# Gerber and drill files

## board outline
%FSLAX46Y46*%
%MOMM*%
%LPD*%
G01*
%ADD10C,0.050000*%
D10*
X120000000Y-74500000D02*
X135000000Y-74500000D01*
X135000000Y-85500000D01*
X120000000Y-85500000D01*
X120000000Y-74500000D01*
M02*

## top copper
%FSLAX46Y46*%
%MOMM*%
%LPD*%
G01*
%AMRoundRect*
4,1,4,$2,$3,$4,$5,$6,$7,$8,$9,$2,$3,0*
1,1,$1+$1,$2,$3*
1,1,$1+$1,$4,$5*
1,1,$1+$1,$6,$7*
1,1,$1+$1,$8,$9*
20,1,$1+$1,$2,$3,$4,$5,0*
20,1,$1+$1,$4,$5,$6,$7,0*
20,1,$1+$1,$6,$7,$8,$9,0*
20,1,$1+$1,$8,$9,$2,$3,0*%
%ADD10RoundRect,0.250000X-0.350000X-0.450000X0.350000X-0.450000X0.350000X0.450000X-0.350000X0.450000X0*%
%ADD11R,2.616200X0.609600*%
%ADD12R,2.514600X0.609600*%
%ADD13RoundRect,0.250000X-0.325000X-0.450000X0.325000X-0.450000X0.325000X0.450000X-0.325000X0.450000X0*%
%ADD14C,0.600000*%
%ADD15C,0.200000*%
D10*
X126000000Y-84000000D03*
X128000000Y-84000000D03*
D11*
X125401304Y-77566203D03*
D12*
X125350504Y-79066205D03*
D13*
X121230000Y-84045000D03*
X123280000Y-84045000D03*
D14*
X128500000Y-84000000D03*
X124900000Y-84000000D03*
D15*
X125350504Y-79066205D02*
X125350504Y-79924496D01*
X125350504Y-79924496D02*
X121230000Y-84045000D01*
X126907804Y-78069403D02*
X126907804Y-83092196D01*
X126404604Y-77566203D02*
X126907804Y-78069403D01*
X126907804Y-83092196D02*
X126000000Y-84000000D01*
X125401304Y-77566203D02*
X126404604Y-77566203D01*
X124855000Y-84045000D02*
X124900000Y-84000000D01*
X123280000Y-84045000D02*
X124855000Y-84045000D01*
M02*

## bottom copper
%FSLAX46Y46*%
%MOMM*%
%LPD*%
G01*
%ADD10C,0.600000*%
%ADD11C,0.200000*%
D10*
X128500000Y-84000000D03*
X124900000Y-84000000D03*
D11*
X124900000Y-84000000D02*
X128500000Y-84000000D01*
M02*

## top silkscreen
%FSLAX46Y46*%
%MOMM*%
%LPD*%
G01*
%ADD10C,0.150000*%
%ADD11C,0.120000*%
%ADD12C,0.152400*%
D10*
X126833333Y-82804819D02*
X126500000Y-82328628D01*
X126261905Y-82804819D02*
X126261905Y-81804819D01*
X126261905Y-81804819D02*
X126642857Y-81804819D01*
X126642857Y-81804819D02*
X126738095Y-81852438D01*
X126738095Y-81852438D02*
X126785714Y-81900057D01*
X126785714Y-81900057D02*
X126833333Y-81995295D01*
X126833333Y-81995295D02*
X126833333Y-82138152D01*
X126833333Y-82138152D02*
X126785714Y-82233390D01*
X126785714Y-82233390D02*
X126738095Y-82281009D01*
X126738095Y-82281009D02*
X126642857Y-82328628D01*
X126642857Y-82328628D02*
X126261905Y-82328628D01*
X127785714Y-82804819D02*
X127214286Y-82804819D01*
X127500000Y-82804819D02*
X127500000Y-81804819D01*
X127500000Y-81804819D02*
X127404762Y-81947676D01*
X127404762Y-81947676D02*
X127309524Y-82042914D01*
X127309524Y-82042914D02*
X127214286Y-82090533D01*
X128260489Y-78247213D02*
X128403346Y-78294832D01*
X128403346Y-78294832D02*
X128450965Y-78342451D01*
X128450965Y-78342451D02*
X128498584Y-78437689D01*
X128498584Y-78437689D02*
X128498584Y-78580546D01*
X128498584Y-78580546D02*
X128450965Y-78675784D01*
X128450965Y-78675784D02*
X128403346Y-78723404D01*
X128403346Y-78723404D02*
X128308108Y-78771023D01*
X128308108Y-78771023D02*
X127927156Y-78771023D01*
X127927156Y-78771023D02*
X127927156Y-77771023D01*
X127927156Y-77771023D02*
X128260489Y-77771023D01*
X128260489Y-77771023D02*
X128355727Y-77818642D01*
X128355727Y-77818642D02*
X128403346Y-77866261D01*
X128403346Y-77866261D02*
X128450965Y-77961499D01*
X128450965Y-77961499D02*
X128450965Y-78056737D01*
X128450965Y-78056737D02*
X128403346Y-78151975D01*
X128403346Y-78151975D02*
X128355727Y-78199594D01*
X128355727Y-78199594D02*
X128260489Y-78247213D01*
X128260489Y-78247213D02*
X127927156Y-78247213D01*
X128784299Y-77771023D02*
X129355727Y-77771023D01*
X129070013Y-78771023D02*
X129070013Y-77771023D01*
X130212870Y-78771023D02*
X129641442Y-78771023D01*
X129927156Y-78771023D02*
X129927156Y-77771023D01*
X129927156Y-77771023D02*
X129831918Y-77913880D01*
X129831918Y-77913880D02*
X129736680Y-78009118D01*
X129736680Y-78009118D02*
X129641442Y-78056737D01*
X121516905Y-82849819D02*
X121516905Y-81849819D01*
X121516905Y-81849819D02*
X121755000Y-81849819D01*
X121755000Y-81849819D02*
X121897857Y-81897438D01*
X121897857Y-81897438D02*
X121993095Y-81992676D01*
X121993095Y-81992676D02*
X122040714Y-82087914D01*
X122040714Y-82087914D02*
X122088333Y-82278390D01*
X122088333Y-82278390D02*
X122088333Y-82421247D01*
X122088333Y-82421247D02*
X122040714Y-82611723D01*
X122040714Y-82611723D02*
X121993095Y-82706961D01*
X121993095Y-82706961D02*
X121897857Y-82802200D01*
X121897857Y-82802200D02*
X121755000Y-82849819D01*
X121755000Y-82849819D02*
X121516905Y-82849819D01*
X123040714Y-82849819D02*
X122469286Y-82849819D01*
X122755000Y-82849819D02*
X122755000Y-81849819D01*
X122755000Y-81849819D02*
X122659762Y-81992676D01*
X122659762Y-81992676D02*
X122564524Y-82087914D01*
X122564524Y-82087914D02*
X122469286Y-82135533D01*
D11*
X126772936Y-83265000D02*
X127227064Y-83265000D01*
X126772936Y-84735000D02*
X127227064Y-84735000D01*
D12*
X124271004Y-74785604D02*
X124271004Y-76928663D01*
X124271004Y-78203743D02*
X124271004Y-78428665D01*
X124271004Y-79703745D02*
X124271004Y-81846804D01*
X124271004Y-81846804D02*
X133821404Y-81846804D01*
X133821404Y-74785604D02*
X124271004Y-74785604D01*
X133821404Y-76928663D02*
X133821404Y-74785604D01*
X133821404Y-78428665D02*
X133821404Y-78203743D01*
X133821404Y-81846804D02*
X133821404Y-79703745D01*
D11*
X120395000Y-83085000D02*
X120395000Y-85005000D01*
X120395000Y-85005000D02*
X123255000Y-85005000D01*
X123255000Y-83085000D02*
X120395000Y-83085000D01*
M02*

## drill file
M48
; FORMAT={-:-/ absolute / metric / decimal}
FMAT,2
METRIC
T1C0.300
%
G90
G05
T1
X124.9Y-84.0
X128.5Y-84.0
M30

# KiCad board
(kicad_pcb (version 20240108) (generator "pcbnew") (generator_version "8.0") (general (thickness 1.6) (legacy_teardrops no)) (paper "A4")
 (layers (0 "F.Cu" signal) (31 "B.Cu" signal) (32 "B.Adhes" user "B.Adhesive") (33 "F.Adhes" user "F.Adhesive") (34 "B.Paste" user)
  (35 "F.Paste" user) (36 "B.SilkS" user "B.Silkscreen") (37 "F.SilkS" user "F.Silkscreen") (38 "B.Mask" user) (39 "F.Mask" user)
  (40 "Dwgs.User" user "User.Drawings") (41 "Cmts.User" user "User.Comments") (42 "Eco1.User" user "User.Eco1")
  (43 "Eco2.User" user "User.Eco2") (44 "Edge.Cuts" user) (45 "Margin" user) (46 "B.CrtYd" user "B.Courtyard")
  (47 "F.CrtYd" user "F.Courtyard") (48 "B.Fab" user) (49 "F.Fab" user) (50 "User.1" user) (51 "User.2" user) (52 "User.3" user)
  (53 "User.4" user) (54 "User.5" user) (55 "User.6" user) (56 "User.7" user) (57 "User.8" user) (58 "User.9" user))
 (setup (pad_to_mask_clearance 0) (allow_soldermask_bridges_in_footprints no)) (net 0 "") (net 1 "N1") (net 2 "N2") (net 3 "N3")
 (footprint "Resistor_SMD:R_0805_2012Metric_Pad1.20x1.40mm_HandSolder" (layer "F.Cu") (at 127 84)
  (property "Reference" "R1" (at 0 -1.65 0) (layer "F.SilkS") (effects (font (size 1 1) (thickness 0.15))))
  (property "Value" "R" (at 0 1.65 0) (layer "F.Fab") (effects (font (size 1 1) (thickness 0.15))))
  (fp_line (start -0.227064 -0.735) (end 0.227064 -0.735) (stroke (width 0.12) (type solid)) (layer "F.SilkS"))
  (fp_line (start -0.227064 0.735) (end 0.227064 0.735) (stroke (width 0.12) (type solid)) (layer "F.SilkS"))
  (pad "1" smd roundrect (at -1 0) (size 1.2 1.4) (layers "F.Cu" "F.Paste" "F.Mask") (roundrect_rratio 0.208333) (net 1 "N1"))
  (pad "2" smd roundrect (at 1 0) (size 1.2 1.4) (layers "F.Cu" "F.Paste" "F.Mask") (roundrect_rratio 0.208333) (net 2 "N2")))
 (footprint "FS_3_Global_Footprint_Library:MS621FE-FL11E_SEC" (layer "F.Cu") (at 129.046204 78.316204)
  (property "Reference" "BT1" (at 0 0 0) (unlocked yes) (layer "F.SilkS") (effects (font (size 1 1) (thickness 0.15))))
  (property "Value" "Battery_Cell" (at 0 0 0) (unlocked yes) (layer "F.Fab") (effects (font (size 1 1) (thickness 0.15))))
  (fp_line (start -4.7752 -3.5306) (end -4.7752 -1.387541) (stroke (width 0.1524) (type solid)) (layer "F.SilkS"))
  (fp_line (start -4.7752 -0.112461) (end -4.7752 0.112461) (stroke (width 0.1524) (type solid)) (layer "F.SilkS"))
  (fp_line (start -4.7752 1.387541) (end -4.7752 3.5306) (stroke (width 0.1524) (type solid)) (layer "F.SilkS"))
  (fp_line (start -4.7752 3.5306) (end 4.7752 3.5306) (stroke (width 0.1524) (type solid)) (layer "F.SilkS"))
  (fp_line (start 4.7752 -3.5306) (end -4.7752 -3.5306) (stroke (width 0.1524) (type solid)) (layer "F.SilkS"))
  (fp_line (start 4.7752 -1.387541) (end 4.7752 -3.5306) (stroke (width 0.1524) (type solid)) (layer "F.SilkS"))
  (fp_line (start 4.7752 0.112461) (end 4.7752 -0.112461) (stroke (width 0.1524) (type solid)) (layer "F.SilkS"))
  (fp_line (start 4.7752 3.5306) (end 4.7752 1.387541) (stroke (width 0.1524) (type solid)) (layer "F.SilkS"))
  (pad "1" smd rect (at -3.6449 -0.750001) (size 2.6162 0.6096) (layers "F.Cu" "F.Paste" "F.Mask") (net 1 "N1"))
  (pad "2" smd rect (at -3.6957 0.750001) (size 2.5146 0.6096) (layers "F.Cu" "F.Paste" "F.Mask") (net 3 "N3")))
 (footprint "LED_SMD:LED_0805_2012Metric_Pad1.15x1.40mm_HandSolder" (layer "F.Cu") (at 122.255 84.045)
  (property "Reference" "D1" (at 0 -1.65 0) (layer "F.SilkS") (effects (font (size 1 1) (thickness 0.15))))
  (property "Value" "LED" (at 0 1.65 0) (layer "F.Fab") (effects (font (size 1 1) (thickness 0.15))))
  (fp_line (start -1.86 -0.96) (end -1.86 0.96) (stroke (width 0.12) (type solid)) (layer "F.SilkS"))
  (fp_line (start -1.86 0.96) (end 1 0.96) (stroke (width 0.12) (type solid)) (layer "F.SilkS"))
  (fp_line (start 1 -0.96) (end -1.86 -0.96) (stroke (width 0.12) (type solid)) (layer "F.SilkS"))
  (pad "1" smd roundrect (at -1.025 0) (size 1.15 1.4) (layers "F.Cu" "F.Paste" "F.Mask") (roundrect_rratio 0.217391) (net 3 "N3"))
  (pad "2" smd roundrect (at 1.025 0) (size 1.15 1.4) (layers "F.Cu" "F.Paste" "F.Mask") (roundrect_rratio 0.217391) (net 2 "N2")))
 (gr_rect (start 120 74.5) (end 135 85.5) (stroke (width 0.05) (type default)) (fill none) (layer "Edge.Cuts"))
 (segment (start 125.350504 79.066205) (end 125.350504 79.924496) (width 0.2) (layer "F.Cu") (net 3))
 (segment (start 125.350504 79.924496) (end 121.23 84.045) (width 0.2) (layer "F.Cu") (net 3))
 (segment (start 126.907804 78.069403) (end 126.907804 83.092196) (width 0.2) (layer "F.Cu") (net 1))
 (segment (start 126.404604 77.566203) (end 126.907804 78.069403) (width 0.2) (layer "F.Cu") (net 1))
 (segment (start 126.907804 83.092196) (end 126 84) (width 0.2) (layer "F.Cu") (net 1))
 (segment (start 125.401304 77.566203) (end 126.404604 77.566203) (width 0.2) (layer "F.Cu") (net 1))
 (segment (start 124.855 84.045) (end 124.9 84) (width 0.2) (layer "F.Cu") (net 2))
 (segment (start 123.28 84.045) (end 124.855 84.045) (width 0.2) (layer "F.Cu") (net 2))
 (via (at 128.5 84) (size 0.6) (drill 0.3) (layers "F.Cu" "B.Cu") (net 2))
 (via (at 124.9 84) (size 0.6) (drill 0.3) (layers "F.Cu" "B.Cu") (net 2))
 (segment (start 124.9 84) (end 128.5 84) (width 0.2) (layer "B.Cu") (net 2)))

